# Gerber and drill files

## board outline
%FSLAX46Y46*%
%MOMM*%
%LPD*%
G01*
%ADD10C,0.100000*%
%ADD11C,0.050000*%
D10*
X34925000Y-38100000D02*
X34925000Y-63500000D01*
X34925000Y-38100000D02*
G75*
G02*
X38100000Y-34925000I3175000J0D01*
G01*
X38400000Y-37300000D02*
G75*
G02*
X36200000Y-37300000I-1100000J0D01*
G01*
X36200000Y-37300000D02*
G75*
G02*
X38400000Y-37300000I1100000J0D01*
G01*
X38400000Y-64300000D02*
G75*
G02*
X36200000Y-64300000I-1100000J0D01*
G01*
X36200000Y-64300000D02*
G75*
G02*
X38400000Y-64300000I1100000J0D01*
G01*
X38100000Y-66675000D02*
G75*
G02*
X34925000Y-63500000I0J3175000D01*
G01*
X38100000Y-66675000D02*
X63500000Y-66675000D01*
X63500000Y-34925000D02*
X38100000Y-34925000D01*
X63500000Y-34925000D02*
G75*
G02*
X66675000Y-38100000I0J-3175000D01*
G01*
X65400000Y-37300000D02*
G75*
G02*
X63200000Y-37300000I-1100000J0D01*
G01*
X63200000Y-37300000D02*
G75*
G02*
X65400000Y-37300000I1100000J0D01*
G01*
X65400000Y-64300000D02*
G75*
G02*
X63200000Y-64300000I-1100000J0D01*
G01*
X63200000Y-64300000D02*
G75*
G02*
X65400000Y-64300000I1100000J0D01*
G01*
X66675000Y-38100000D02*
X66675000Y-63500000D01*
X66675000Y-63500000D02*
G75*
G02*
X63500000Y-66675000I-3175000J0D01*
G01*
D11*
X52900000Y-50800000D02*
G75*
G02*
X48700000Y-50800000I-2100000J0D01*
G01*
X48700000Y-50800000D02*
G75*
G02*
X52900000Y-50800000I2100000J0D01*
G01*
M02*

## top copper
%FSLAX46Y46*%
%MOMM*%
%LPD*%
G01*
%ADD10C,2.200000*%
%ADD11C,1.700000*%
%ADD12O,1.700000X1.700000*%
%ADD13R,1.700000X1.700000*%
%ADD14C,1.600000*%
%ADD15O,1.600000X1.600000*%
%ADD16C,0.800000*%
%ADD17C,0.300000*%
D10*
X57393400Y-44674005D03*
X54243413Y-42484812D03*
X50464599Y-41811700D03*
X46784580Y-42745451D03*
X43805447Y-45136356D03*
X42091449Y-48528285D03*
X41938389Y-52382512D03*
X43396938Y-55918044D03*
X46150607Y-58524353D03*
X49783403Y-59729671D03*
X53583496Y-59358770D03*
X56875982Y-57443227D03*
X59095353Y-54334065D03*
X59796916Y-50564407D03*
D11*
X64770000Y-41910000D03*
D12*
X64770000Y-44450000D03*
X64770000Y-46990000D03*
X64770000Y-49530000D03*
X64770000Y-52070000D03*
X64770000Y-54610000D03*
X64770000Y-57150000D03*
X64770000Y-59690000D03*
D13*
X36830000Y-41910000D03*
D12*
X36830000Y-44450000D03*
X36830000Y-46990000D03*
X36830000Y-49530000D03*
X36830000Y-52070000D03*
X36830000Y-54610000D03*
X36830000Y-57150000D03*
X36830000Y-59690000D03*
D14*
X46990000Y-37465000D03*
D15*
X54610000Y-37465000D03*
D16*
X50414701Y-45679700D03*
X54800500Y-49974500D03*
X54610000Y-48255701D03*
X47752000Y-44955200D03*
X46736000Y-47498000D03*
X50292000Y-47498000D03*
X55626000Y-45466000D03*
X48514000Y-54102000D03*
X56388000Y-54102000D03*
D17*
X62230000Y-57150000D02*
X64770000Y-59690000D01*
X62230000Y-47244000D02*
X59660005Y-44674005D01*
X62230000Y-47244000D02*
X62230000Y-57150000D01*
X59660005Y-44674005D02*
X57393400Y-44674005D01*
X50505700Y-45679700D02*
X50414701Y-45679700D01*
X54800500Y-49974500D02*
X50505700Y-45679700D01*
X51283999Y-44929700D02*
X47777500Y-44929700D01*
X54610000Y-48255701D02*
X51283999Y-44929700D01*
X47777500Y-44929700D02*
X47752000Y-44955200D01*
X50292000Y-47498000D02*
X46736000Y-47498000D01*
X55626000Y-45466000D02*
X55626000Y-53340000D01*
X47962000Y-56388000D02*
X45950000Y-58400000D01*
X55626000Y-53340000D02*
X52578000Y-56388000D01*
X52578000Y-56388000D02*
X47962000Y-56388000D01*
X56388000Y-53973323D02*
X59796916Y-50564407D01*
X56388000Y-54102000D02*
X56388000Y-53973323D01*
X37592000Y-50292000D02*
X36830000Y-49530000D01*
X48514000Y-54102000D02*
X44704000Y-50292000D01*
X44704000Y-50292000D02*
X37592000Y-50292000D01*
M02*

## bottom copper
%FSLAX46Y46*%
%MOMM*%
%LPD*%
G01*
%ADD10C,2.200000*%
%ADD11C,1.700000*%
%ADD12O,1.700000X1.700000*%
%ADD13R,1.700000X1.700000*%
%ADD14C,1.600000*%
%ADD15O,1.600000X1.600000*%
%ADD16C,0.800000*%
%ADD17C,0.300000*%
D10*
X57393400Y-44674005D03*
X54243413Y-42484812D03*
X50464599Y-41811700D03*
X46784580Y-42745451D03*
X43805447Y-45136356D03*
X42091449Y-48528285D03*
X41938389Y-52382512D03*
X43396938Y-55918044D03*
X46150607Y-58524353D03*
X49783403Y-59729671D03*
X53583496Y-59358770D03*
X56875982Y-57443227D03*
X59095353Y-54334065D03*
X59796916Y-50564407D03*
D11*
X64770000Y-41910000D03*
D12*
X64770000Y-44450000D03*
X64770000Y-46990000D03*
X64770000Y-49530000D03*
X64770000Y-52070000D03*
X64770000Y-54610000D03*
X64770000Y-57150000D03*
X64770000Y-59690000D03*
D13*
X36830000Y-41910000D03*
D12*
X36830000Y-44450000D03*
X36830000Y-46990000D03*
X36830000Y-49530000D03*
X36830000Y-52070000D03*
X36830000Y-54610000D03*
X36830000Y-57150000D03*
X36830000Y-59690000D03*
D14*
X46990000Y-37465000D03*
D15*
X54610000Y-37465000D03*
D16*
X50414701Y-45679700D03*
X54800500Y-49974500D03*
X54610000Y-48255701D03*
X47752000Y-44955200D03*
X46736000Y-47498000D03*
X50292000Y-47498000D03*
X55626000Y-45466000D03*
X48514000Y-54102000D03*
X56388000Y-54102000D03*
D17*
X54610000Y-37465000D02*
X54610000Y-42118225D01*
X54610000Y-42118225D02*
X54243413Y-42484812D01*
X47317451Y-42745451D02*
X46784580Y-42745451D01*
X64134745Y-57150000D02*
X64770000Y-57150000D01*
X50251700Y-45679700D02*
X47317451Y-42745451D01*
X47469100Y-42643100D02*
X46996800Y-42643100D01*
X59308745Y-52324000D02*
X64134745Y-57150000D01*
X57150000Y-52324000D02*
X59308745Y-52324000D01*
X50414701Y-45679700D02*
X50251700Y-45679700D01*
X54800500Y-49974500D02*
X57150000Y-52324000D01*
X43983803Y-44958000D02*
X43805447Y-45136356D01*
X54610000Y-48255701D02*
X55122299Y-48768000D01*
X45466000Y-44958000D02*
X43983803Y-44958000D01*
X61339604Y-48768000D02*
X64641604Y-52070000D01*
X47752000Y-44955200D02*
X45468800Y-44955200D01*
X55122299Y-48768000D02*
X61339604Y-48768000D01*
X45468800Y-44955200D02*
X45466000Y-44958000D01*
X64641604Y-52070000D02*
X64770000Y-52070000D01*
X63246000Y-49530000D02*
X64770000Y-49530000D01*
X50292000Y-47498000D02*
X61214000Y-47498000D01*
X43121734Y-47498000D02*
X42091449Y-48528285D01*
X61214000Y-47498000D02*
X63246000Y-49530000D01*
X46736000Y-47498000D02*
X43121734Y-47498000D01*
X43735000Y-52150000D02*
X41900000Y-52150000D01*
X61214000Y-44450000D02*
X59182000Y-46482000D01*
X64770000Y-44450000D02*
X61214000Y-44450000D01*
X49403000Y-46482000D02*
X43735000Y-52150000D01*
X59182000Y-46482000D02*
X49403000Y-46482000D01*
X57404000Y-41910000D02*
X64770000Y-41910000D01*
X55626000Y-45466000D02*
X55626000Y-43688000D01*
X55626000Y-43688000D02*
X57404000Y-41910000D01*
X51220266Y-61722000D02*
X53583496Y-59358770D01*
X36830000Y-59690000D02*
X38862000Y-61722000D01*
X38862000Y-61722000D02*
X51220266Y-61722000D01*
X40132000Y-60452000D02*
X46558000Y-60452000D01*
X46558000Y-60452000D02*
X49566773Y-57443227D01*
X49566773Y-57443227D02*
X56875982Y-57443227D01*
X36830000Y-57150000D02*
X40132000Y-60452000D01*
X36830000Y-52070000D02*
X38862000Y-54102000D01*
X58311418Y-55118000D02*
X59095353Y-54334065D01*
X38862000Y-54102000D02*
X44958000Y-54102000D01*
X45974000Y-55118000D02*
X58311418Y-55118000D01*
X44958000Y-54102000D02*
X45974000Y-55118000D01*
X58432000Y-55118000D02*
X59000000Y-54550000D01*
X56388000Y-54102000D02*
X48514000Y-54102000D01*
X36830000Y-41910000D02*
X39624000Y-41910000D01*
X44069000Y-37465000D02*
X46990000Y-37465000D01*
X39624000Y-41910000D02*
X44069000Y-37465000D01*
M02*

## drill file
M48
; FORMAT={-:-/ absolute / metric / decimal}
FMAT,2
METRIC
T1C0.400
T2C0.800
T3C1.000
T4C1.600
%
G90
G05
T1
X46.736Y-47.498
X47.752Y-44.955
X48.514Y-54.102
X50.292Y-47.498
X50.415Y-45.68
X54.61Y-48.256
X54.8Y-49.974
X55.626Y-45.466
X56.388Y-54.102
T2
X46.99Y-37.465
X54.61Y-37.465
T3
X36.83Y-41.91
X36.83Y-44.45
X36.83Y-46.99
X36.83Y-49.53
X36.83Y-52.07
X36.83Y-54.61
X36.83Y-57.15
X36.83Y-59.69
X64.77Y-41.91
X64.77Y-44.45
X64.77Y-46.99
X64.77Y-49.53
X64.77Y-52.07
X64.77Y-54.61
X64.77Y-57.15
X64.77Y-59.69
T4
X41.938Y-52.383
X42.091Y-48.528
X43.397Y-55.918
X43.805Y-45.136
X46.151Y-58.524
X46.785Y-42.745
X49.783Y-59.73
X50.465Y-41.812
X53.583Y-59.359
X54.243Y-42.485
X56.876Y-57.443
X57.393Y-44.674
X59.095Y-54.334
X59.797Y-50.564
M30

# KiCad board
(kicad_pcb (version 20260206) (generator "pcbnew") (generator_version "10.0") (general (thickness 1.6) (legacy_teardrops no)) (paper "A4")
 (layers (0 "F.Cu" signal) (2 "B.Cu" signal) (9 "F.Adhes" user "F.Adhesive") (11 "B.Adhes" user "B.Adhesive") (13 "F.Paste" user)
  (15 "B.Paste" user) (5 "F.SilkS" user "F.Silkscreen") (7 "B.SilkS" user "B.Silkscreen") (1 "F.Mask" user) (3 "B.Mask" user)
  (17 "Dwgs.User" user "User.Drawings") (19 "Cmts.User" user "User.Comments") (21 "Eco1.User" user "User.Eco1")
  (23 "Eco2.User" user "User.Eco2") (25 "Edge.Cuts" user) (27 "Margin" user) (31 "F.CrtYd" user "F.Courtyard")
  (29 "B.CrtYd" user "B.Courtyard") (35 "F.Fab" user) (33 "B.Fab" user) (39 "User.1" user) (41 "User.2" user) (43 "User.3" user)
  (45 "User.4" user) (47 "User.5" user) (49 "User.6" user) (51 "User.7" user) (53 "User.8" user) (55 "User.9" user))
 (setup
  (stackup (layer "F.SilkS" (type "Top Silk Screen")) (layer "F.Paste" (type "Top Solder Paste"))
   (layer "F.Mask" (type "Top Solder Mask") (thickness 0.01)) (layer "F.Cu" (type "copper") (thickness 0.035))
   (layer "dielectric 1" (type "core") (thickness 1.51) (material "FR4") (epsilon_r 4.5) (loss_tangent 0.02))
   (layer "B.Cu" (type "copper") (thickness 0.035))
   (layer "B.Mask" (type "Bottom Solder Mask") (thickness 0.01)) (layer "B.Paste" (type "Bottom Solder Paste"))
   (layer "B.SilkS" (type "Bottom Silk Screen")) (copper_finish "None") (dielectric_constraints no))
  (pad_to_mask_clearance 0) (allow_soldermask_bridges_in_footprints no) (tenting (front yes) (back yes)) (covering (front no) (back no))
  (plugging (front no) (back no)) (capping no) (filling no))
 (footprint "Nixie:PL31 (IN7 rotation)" (layer "F.Cu") (at 50.8 50.8 90)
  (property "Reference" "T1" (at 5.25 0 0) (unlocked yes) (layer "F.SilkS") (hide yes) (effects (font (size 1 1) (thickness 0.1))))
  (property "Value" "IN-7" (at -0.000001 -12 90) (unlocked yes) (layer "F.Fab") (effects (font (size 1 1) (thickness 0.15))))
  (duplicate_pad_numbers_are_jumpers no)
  (fp_circle (center 0 0) (end 2.1 0) (stroke (width 0.05) (type default)) (fill no) (layer "Edge.Cuts"))
  (pad "1" thru_hole circle (at 6.125995 6.5934 271.5) (size 2.2 2.2) (drill 1.6) (layers "*.Cu" "*.Mask") (remove_unused_layers no)
   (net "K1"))
  (pad "2" thru_hole circle (at 8.315188 3.443413 271.5) (size 2.2 2.2) (drill 1.6) (layers "*.Cu" "*.Mask") (remove_unused_layers no)
   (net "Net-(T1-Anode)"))
  (pad "3" thru_hole circle (at 8.9883 -0.335401 271.5) (size 2.2 2.2) (drill 1.6) (layers "*.Cu" "*.Mask") (remove_unused_layers no)
   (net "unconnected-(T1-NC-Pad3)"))
  (pad "4" thru_hole circle (at 8.054549 -4.01542 271.5) (size 2.2 2.2) (drill 1.6) (layers "*.Cu" "*.Mask") (remove_unused_layers no)
   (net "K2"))
  (pad "5" thru_hole circle (at 5.663644 -6.994553 271.5) (size 2.2 2.2) (drill 1.6) (layers "*.Cu" "*.Mask") (remove_unused_layers no)
   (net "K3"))
  (pad "6" thru_hole circle (at 2.271715 -8.708551 271.5) (size 2.2 2.2) (drill 1.6) (layers "*.Cu" "*.Mask") (remove_unused_layers no)
   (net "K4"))
  (pad "7" thru_hole circle (at -1.582512 -8.861611 271.5) (size 2.2 2.2) (drill 1.6) (layers "*.Cu" "*.Mask") (remove_unused_layers no)
   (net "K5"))
  (pad "8" thru_hole circle (at -5.118044 -7.403062 271.5) (size 2.2 2.2) (drill 1.6) (layers "*.Cu" "*.Mask") (remove_unused_layers no)
   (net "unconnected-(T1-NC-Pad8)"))
  (pad "9" thru_hole circle (at -7.724353 -4.649393 271.5) (size 2.2 2.2) (drill 1.6) (layers "*.Cu" "*.Mask") (remove_unused_layers no)
   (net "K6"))
  (pad "10" thru_hole circle (at -8.929671 -1.016597 271.5) (size 2.2 2.2) (drill 1.6) (layers "*.Cu" "*.Mask") (remove_unused_layers no)
   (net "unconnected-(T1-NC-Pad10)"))
  (pad "11" thru_hole circle (at -8.55877 2.783496 271.5) (size 2.2 2.2) (drill 1.6) (layers "*.Cu" "*.Mask") (remove_unused_layers no)
   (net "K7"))
  (pad "12" thru_hole circle (at -6.643227 6.075982 271.5) (size 2.2 2.2) (drill 1.6) (layers "*.Cu" "*.Mask") (remove_unused_layers no)
   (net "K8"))
  (pad "13" thru_hole circle (at -3.534065 8.295353 271.5) (size 2.2 2.2) (drill 1.6) (layers "*.Cu" "*.Mask") (remove_unused_layers no)
   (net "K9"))
  (pad "14" thru_hole circle (at 0.235593 8.996916 271.5) (size 2.2 2.2) (drill 1.6) (layers "*.Cu" "*.Mask") (remove_unused_layers no)
   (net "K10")))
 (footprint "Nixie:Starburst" (layer "F.Cu") (at 43 63.25)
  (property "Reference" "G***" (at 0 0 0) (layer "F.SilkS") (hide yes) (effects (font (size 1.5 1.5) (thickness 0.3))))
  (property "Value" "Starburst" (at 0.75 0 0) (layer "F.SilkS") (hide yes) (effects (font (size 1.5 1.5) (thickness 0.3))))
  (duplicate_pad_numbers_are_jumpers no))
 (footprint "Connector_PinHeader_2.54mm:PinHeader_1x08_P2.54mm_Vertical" (layer "B.Cu") (at 64.77 41.91 180)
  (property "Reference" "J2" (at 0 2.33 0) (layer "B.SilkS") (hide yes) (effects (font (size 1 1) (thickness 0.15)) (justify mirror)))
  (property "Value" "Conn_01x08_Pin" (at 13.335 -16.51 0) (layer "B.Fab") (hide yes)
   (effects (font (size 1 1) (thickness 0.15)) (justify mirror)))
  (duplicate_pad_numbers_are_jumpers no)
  (pad "1" thru_hole circle (at 0 0 180) (size 1.7 1.7) (drill 1) (layers "*.Cu" "*.Mask") (remove_unused_layers no) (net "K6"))
  (pad "2" thru_hole oval (at 0 -2.54 180) (size 1.7 1.7) (drill 1) (layers "*.Cu" "*.Mask") (remove_unused_layers no) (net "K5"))
  (pad "3" thru_hole oval (at 0 -5.08 180) (size 1.7 1.7) (drill 1) (layers "*.Cu" "*.Mask") (remove_unused_layers no)
   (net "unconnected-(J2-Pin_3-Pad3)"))
  (pad "4" thru_hole oval (at 0 -7.62 180) (size 1.7 1.7) (drill 1) (layers "*.Cu" "*.Mask") (remove_unused_layers no) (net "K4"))
  (pad "5" thru_hole oval (at 0 -10.16 180) (size 1.7 1.7) (drill 1) (layers "*.Cu" "*.Mask") (remove_unused_layers no) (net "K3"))
  (pad "6" thru_hole oval (at 0 -12.7 180) (size 1.7 1.7) (drill 1) (layers "*.Cu" "*.Mask") (remove_unused_layers no)
   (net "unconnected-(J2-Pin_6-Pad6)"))
  (pad "7" thru_hole oval (at 0 -15.24 180) (size 1.7 1.7) (drill 1) (layers "*.Cu" "*.Mask") (remove_unused_layers no) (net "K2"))
  (pad "8" thru_hole oval (at 0 -17.78 180) (size 1.7 1.7) (drill 1) (layers "*.Cu" "*.Mask") (remove_unused_layers no) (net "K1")))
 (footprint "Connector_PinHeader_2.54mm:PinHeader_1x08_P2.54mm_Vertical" (layer "B.Cu") (at 36.83 41.91 180)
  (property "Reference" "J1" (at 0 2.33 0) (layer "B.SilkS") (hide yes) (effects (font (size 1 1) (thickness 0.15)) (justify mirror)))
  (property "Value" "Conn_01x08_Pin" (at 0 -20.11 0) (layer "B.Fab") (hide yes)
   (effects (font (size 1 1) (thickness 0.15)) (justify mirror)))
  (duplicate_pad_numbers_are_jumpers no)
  (pad "1" thru_hole rect (at 0 0 180) (size 1.7 1.7) (drill 1) (layers "*.Cu" "*.Mask") (remove_unused_layers no) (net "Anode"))
  (pad "2" thru_hole oval (at 0 -2.54 180) (size 1.7 1.7) (drill 1) (layers "*.Cu" "*.Mask") (remove_unused_layers no)
   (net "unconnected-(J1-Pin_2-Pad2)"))
  (pad "3" thru_hole oval (at 0 -5.08 180) (size 1.7 1.7) (drill 1) (layers "*.Cu" "*.Mask") (remove_unused_layers no)
   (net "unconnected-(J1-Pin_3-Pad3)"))
  (pad "4" thru_hole oval (at 0 -7.62 180) (size 1.7 1.7) (drill 1) (layers "*.Cu" "*.Mask") (remove_unused_layers no) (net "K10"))
  (pad "5" thru_hole oval (at 0 -10.16 180) (size 1.7 1.7) (drill 1) (layers "*.Cu" "*.Mask") (remove_unused_layers no) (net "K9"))
  (pad "6" thru_hole oval (at 0 -12.7 180) (size 1.7 1.7) (drill 1) (layers "*.Cu" "*.Mask") (remove_unused_layers no)
   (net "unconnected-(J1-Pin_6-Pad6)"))
  (pad "7" thru_hole oval (at 0 -15.24 180) (size 1.7 1.7) (drill 1) (layers "*.Cu" "*.Mask") (remove_unused_layers no) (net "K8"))
  (pad "8" thru_hole oval (at 0 -17.78 180) (size 1.7 1.7) (drill 1) (layers "*.Cu" "*.Mask") (remove_unused_layers no) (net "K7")))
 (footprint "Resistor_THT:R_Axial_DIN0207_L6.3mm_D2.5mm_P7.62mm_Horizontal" (layer "B.Cu") (at 46.99 37.465)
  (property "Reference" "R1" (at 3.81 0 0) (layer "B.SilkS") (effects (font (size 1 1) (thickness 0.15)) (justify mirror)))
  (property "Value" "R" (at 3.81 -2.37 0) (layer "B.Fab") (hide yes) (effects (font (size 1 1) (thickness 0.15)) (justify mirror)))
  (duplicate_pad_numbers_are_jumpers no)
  (pad "1" thru_hole circle (at 0 0) (size 1.6 1.6) (drill 0.8) (layers "*.Cu" "*.Mask") (remove_unused_layers no) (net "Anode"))
  (pad "2" thru_hole oval (at 7.62 0) (size 1.6 1.6) (drill 0.8) (layers "*.Cu" "*.Mask") (remove_unused_layers no) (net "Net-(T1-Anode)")))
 (gr_line (start 34.925 38.1) (end 34.925 63.5) (stroke (width 0.1) (type default)) (layer "Edge.Cuts"))
 (gr_arc (start 34.925 38.1) (mid 35.854936 35.854936) (end 38.1 34.925) (stroke (width 0.1) (type default)) (layer "Edge.Cuts"))
 (gr_circle (center 37.3 37.3) (end 38.4 37.3) (stroke (width 0.1) (type default)) (fill no) (layer "Edge.Cuts"))
 (gr_circle (center 37.3 64.3) (end 38.4 64.3) (stroke (width 0.1) (type default)) (fill no) (layer "Edge.Cuts"))
 (gr_arc (start 38.1 66.675) (mid 35.854936 65.745064) (end 34.925 63.5) (stroke (width 0.1) (type default)) (layer "Edge.Cuts"))
 (gr_line (start 38.1 66.675) (end 63.5 66.675) (stroke (width 0.1) (type default)) (layer "Edge.Cuts"))
 (gr_line (start 63.5 34.925) (end 38.1 34.925) (stroke (width 0.1) (type default)) (layer "Edge.Cuts"))
 (gr_arc (start 63.5 34.925) (mid 65.745064 35.854936) (end 66.675 38.1) (stroke (width 0.1) (type default)) (layer "Edge.Cuts"))
 (gr_circle (center 64.3 37.3) (end 65.4 37.3) (stroke (width 0.1) (type default)) (fill no) (layer "Edge.Cuts"))
 (gr_circle (center 64.3 64.3) (end 65.4 64.3) (stroke (width 0.1) (type default)) (fill no) (layer "Edge.Cuts"))
 (gr_line (start 66.675 38.1) (end 66.675 63.5) (stroke (width 0.1) (type default)) (layer "Edge.Cuts"))
 (gr_arc (start 66.675 63.5) (mid 65.745064 65.745064) (end 63.5 66.675) (stroke (width 0.1) (type default)) (layer "Edge.Cuts"))
 (segment (start 62.23 57.15) (end 64.77 59.69) (width 0.3) (layer "F.Cu") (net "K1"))
 (segment (start 62.23 47.244) (end 59.660005 44.674005) (width 0.3) (layer "F.Cu") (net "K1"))
 (segment (start 62.23 47.244) (end 62.23 57.15) (width 0.3) (layer "F.Cu") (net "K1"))
 (segment (start 59.660005 44.674005) (end 57.3934 44.674005) (width 0.3) (layer "F.Cu") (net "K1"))
 (segment (start 54.61 37.465) (end 54.61 42.118225) (width 0.3) (layer "B.Cu") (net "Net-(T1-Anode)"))
 (segment (start 54.61 42.118225) (end 54.243413 42.484812) (width 0.3) (layer "B.Cu") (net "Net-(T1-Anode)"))
 (segment (start 50.5057 45.6797) (end 50.414701 45.6797) (width 0.3) (layer "F.Cu") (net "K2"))
 (segment (start 54.8005 49.9745) (end 50.5057 45.6797) (width 0.3) (layer "F.Cu") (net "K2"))
 (via (at 50.414701 45.6797) (size 0.8) (drill 0.4) (layers "F.Cu" "B.Cu") (capping no) (covering (front no) (back no))
  (plugging (front no) (back no)) (filling no) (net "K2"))
 (via (at 54.8005 49.9745) (size 0.8) (drill 0.4) (layers "F.Cu" "B.Cu") (capping no) (covering (front no) (back no))
  (plugging (front no) (back no)) (filling no) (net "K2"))
 (segment (start 47.317451 42.745451) (end 46.78458 42.745451) (width 0.3) (layer "B.Cu") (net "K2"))
 (segment (start 64.134745 57.15) (end 64.77 57.15) (width 0.3) (layer "B.Cu") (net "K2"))
 (segment (start 50.2517 45.6797) (end 47.317451 42.745451) (width 0.3) (layer "B.Cu") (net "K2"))
 (segment (start 47.4691 42.6431) (end 46.9968 42.6431) (width 0.3) (layer "B.Cu") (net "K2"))
 (segment (start 59.308745 52.324) (end 64.134745 57.15) (width 0.3) (layer "B.Cu") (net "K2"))
 (segment (start 57.15 52.324) (end 59.308745 52.324) (width 0.3) (layer "B.Cu") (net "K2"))
 (segment (start 50.414701 45.6797) (end 50.2517 45.6797) (width 0.3) (layer "B.Cu") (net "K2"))
 (segment (start 54.8005 49.9745) (end 57.15 52.324) (width 0.3) (layer "B.Cu") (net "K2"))
 (segment (start 51.283999 44.9297) (end 47.7775 44.9297) (width 0.3) (layer "F.Cu") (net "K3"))
 (segment (start 54.61 48.255701) (end 51.283999 44.9297) (width 0.3) (layer "F.Cu") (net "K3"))
 (segment (start 47.7775 44.9297) (end 47.752 44.9552) (width 0.3) (layer "F.Cu") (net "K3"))
 (via (at 54.61 48.255701) (size 0.8) (drill 0.4) (layers "F.Cu" "B.Cu") (capping no) (covering (front no) (back no))
  (plugging (front no) (back no)) (filling no) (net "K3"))
 (via (at 47.752 44.9552) (size 0.8) (drill 0.4) (layers "F.Cu" "B.Cu") (capping no) (covering (front no) (back no))
  (plugging (front no) (back no)) (filling no) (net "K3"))
 (segment (start 43.983803 44.958) (end 43.805447 45.136356) (width 0.3) (layer "B.Cu") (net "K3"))
 (segment (start 54.61 48.255701) (end 55.122299 48.768) (width 0.3) (layer "B.Cu") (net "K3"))
 (segment (start 45.466 44.958) (end 43.983803 44.958) (width 0.3) (layer "B.Cu") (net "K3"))
 (segment (start 61.339604 48.768) (end 64.641604 52.07) (width 0.3) (layer "B.Cu") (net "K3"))
 (segment (start 47.752 44.9552) (end 45.4688 44.9552) (width 0.3) (layer "B.Cu") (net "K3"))
 (segment (start 55.122299 48.768) (end 61.339604 48.768) (width 0.3) (layer "B.Cu") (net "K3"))
 (segment (start 45.4688 44.9552) (end 45.466 44.958) (width 0.3) (layer "B.Cu") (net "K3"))
 (segment (start 64.641604 52.07) (end 64.77 52.07) (width 0.3) (layer "B.Cu") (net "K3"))
 (segment (start 50.292 47.498) (end 46.736 47.498) (width 0.3) (layer "F.Cu") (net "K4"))
 (via (at 46.736 47.498) (size 0.8) (drill 0.4) (layers "F.Cu" "B.Cu") (capping no) (covering (front no) (back no))
  (plugging (front no) (back no)) (filling no) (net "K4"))
 (via (at 50.292 47.498) (size 0.8) (drill 0.4) (layers "F.Cu" "B.Cu") (capping no) (covering (front no) (back no))
  (plugging (front no) (back no)) (filling no) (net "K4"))
 (segment (start 63.246 49.53) (end 64.77 49.53) (width 0.3) (layer "B.Cu") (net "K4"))
 (segment (start 50.292 47.498) (end 61.214 47.498) (width 0.3) (layer "B.Cu") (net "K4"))
 (segment (start 43.121734 47.498) (end 42.091449 48.528285) (width 0.3) (layer "B.Cu") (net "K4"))
 (segment (start 61.214 47.498) (end 63.246 49.53) (width 0.3) (layer "B.Cu") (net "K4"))
 (segment (start 46.736 47.498) (end 43.121734 47.498) (width 0.3) (layer "B.Cu") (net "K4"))
 (segment (start 43.735 52.15) (end 41.9 52.15) (width 0.3) (layer "B.Cu") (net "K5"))
 (segment (start 61.214 44.45) (end 59.182 46.482) (width 0.3) (layer "B.Cu") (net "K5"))
 (segment (start 64.77 44.45) (end 61.214 44.45) (width 0.3) (layer "B.Cu") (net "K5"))
 (segment (start 49.403 46.482) (end 43.735 52.15) (width 0.3) (layer "B.Cu") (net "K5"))
 (segment (start 59.182 46.482) (end 49.403 46.482) (width 0.3) (layer "B.Cu") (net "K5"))
 (segment (start 55.626 45.466) (end 55.626 53.34) (width 0.3) (layer "F.Cu") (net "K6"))
 (segment (start 47.962 56.388) (end 45.95 58.4) (width 0.3) (layer "F.Cu") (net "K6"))
 (segment (start 55.626 53.34) (end 52.578 56.388) (width 0.3) (layer "F.Cu") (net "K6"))
 (segment (start 52.578 56.388) (end 47.962 56.388) (width 0.3) (layer "F.Cu") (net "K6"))
 (via (at 55.626 45.466) (size 0.8) (drill 0.4) (layers "F.Cu" "B.Cu") (capping no) (covering (front no) (back no))
  (plugging (front no) (back no)) (filling no) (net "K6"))
 (segment (start 57.404 41.91) (end 64.77 41.91) (width 0.3) (layer "B.Cu") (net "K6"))
 (segment (start 55.626 45.466) (end 55.626 43.688) (width 0.3) (layer "B.Cu") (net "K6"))
 (segment (start 55.626 43.688) (end 57.404 41.91) (width 0.3) (layer "B.Cu") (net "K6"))
 (segment (start 51.220266 61.722) (end 53.583496 59.35877) (width 0.3) (layer "B.Cu") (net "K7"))
 (segment (start 36.83 59.69) (end 38.862 61.722) (width 0.3) (layer "B.Cu") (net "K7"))
 (segment (start 38.862 61.722) (end 51.220266 61.722) (width 0.3) (layer "B.Cu") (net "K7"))
 (segment (start 40.132 60.452) (end 46.558 60.452) (width 0.3) (layer "B.Cu") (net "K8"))
 (segment (start 46.558 60.452) (end 49.566773 57.443227) (width 0.3) (layer "B.Cu") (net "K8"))
 (segment (start 49.566773 57.443227) (end 56.875982 57.443227) (width 0.3) (layer "B.Cu") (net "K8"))
 (segment (start 36.83 57.15) (end 40.132 60.452) (width 0.3) (layer "B.Cu") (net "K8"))
 (segment (start 36.83 52.07) (end 38.862 54.102) (width 0.3) (layer "B.Cu") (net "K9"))
 (segment (start 58.311418 55.118) (end 59.095353 54.334065) (width 0.3) (layer "B.Cu") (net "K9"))
 (segment (start 38.862 54.102) (end 44.958 54.102) (width 0.3) (layer "B.Cu") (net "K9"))
 (segment (start 45.974 55.118) (end 58.311418 55.118) (width 0.3) (layer "B.Cu") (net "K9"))
 (segment (start 44.958 54.102) (end 45.974 55.118) (width 0.3) (layer "B.Cu") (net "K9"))
 (segment (start 58.432 55.118) (end 59 54.55) (width 0.3) (layer "B.Cu") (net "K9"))
 (segment (start 56.388 53.973323) (end 59.796916 50.564407) (width 0.3) (layer "F.Cu") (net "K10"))
 (segment (start 56.388 54.102) (end 56.388 53.973323) (width 0.3) (layer "F.Cu") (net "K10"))
 (segment (start 37.592 50.292) (end 36.83 49.53) (width 0.3) (layer "F.Cu") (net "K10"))
 (segment (start 48.514 54.102) (end 44.704 50.292) (width 0.3) (layer "F.Cu") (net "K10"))
 (segment (start 44.704 50.292) (end 37.592 50.292) (width 0.3) (layer "F.Cu") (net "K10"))
 (via (at 48.514 54.102) (size 0.8) (drill 0.4) (layers "F.Cu" "B.Cu") (capping no) (covering (front no) (back no))
  (plugging (front no) (back no)) (filling no) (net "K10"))
 (via (at 56.388 54.102) (size 0.8) (drill 0.4) (layers "F.Cu" "B.Cu") (capping no) (covering (front no) (back no))
  (plugging (front no) (back no)) (filling no) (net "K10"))
 (segment (start 56.388 54.102) (end 48.514 54.102) (width 0.3) (layer "B.Cu") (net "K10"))
 (segment (start 36.83 41.91) (end 39.624 41.91) (width 0.3) (layer "B.Cu") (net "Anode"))
 (segment (start 44.069 37.465) (end 46.99 37.465) (width 0.3) (layer "B.Cu") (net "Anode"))
 (segment (start 39.624 41.91) (end 44.069 37.465) (width 0.3) (layer "B.Cu") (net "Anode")))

